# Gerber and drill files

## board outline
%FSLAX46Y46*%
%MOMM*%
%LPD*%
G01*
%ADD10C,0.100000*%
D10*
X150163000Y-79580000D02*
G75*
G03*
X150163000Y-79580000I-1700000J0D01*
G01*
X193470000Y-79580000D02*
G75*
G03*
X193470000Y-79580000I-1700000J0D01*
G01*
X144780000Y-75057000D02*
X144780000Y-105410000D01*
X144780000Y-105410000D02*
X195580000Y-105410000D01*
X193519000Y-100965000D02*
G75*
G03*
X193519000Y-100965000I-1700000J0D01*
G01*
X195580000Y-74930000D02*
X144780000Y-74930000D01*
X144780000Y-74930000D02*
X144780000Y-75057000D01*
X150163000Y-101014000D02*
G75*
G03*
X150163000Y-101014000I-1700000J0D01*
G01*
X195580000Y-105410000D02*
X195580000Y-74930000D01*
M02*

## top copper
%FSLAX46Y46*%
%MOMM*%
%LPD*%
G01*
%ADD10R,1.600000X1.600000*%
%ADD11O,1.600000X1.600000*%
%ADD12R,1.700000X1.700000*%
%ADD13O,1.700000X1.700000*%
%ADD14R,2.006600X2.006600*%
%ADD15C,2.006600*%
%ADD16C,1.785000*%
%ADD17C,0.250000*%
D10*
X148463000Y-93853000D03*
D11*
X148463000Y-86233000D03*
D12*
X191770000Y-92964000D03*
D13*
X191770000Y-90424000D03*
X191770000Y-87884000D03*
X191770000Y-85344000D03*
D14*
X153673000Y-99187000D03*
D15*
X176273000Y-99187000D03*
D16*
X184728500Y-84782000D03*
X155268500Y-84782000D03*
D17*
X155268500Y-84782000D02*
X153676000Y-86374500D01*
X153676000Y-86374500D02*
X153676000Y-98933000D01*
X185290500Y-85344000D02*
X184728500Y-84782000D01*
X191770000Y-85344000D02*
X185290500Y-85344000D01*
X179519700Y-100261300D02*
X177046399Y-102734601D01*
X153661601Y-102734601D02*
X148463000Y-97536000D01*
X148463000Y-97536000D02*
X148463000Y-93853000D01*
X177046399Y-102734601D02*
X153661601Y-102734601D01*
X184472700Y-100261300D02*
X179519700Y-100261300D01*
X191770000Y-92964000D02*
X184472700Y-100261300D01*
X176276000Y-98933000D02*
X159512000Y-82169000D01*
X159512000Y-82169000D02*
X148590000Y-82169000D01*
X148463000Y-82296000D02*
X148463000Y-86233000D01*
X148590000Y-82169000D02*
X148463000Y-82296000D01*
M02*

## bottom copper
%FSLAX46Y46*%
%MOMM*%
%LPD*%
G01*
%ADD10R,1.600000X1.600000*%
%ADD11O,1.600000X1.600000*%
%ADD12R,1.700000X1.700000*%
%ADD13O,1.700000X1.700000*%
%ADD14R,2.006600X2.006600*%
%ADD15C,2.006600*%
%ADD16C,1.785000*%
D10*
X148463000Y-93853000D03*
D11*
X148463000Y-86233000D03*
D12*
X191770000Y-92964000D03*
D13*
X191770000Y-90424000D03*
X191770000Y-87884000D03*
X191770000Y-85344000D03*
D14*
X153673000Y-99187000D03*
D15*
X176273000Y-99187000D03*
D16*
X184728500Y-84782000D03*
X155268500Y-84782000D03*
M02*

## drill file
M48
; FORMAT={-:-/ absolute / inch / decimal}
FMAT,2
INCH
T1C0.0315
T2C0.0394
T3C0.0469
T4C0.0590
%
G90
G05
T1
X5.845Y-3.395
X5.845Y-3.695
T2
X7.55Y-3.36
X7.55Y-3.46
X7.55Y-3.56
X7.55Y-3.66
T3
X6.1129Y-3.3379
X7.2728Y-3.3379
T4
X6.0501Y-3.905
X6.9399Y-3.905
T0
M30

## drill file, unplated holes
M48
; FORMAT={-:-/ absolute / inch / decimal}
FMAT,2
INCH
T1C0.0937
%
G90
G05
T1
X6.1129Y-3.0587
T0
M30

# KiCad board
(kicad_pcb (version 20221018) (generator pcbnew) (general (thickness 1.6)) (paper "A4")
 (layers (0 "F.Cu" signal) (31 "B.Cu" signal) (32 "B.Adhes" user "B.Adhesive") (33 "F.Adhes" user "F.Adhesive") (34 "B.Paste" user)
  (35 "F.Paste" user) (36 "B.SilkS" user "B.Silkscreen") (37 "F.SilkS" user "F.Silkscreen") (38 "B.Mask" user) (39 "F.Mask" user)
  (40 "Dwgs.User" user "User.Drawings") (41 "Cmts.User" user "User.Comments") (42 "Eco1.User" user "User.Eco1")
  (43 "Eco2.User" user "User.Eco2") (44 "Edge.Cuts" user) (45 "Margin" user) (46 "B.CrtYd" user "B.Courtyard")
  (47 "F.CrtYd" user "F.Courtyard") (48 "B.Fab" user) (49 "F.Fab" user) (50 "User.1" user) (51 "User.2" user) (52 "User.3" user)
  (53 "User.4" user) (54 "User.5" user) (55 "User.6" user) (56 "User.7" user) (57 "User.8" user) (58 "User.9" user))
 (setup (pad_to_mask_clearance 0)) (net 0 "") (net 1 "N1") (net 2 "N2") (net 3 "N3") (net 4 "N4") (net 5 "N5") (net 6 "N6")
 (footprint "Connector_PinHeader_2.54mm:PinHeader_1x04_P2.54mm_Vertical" (layer "F.Cu") (at 191.77 92.964 180)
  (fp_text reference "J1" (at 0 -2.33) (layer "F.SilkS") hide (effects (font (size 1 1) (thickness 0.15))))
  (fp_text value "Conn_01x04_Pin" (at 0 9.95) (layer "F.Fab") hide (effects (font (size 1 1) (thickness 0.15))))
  (pad "1" thru_hole rect (at 0 0 180) (size 1.7 1.7) (drill 1) (layers "*.Cu" "*.Mask") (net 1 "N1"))
  (pad "2" thru_hole oval (at 0 2.54 180) (size 1.7 1.7) (drill 1) (layers "*.Cu" "*.Mask") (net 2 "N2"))
  (pad "3" thru_hole oval (at 0 5.08 180) (size 1.7 1.7) (drill 1) (layers "*.Cu" "*.Mask") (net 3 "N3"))
  (pad "4" thru_hole oval (at 0 7.62 180) (size 1.7 1.7) (drill 1) (layers "*.Cu" "*.Mask") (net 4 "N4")))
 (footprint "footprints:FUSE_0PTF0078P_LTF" (layer "F.Cu") (at 153.673 99.187)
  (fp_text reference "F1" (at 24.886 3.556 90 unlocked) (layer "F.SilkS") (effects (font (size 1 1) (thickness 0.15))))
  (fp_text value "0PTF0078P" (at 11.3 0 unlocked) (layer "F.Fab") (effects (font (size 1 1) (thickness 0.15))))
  (pad "1" thru_hole rect (at 0 0) (size 2.0066 2.0066) (drill 1.4986) (layers "*.Cu" "*.Mask") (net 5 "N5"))
  (pad "2" thru_hole circle (at 22.6 0) (size 2.0066 2.0066) (drill 1.4986) (layers "*.Cu" "*.Mask") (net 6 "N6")))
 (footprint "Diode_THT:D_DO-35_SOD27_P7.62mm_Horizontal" (layer "F.Cu") (at 148.463 93.853 90)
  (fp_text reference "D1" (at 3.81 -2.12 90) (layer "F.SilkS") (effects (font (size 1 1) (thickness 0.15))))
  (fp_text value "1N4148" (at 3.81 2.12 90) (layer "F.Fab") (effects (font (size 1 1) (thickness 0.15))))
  (pad "1" thru_hole rect (at 0 0 90) (size 1.6 1.6) (drill 0.8) (layers "*.Cu" "*.Mask") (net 1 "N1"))
  (pad "2" thru_hole oval (at 7.62 0 90) (size 1.6 1.6) (drill 0.8) (layers "*.Cu" "*.Mask") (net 6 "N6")))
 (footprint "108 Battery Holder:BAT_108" (layer "F.Cu") (at 169.9985 84.782)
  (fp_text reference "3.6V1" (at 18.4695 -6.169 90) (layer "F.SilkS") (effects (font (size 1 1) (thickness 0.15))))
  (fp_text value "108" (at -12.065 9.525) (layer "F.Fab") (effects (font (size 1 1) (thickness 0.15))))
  (pad "" np_thru_hole circle (at -14.73 -7.09) (size 2.38 2.38) (drill 2.38) (layers "*.Cu" "*.Mask"))
  (pad "N" thru_hole circle (at 14.73 0) (size 1.785 1.785) (drill 1.19) (layers "*.Cu" "*.Mask") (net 4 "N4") (solder_mask_margin 0.102))
  (pad "P" thru_hole circle (at -14.73 0) (size 1.785 1.785) (drill 1.19) (layers "*.Cu" "*.Mask") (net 5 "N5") (solder_mask_margin 0.102)))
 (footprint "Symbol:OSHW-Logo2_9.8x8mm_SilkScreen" (layer "B.Cu") (at 183.515 98.933 180)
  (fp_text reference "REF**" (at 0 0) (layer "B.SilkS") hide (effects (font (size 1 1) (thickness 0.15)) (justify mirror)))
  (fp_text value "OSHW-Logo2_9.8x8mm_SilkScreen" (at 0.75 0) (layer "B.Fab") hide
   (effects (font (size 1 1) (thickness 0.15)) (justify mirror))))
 (gr_circle (center 148.463 79.58) (end 150.163 79.58) (stroke (width 0.1) (type default)) (fill none) (layer "Edge.Cuts"))
 (gr_circle (center 191.77 79.58) (end 193.47 79.58) (stroke (width 0.1) (type default)) (fill none) (layer "Edge.Cuts"))
 (gr_line (start 144.78 75.057) (end 144.78 105.41) (stroke (width 0.1) (type default)) (layer "Edge.Cuts"))
 (gr_line (start 144.78 105.41) (end 195.58 105.41) (stroke (width 0.1) (type default)) (layer "Edge.Cuts"))
 (gr_circle (center 191.819 100.965) (end 193.519 100.965) (stroke (width 0.1) (type default)) (fill none) (layer "Edge.Cuts"))
 (gr_line (start 195.58 74.93) (end 144.78 74.93) (stroke (width 0.1) (type default)) (layer "Edge.Cuts"))
 (gr_line (start 144.78 74.93) (end 144.78 75.057) (stroke (width 0.1) (type default)) (layer "Edge.Cuts"))
 (gr_circle (center 148.463 101.014) (end 150.163 101.014) (stroke (width 0.1) (type default)) (fill none) (layer "Edge.Cuts"))
 (gr_line (start 195.58 105.41) (end 195.58 74.93) (stroke (width 0.1) (type default)) (layer "Edge.Cuts"))
 (segment (start 155.2685 84.782) (end 153.676 86.3745) (width 0.25) (layer "F.Cu") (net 5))
 (segment (start 153.676 86.3745) (end 153.676 98.933) (width 0.25) (layer "F.Cu") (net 5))
 (segment (start 185.2905 85.344) (end 184.7285 84.782) (width 0.25) (layer "F.Cu") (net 4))
 (segment (start 191.77 85.344) (end 185.2905 85.344) (width 0.25) (layer "F.Cu") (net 4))
 (segment (start 179.5197 100.2613) (end 177.046399 102.734601) (width 0.25) (layer "F.Cu") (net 1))
 (segment (start 153.661601 102.734601) (end 148.463 97.536) (width 0.25) (layer "F.Cu") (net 1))
 (segment (start 148.463 97.536) (end 148.463 93.853) (width 0.25) (layer "F.Cu") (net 1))
 (segment (start 177.046399 102.734601) (end 153.661601 102.734601) (width 0.25) (layer "F.Cu") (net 1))
 (segment (start 184.4727 100.2613) (end 179.5197 100.2613) (width 0.25) (layer "F.Cu") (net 1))
 (segment (start 191.77 92.964) (end 184.4727 100.2613) (width 0.25) (layer "F.Cu") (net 1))
 (segment (start 176.276 98.933) (end 159.512 82.169) (width 0.25) (layer "F.Cu") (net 6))
 (segment (start 159.512 82.169) (end 148.59 82.169) (width 0.25) (layer "F.Cu") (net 6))
 (segment (start 148.463 82.296) (end 148.463 86.233) (width 0.25) (layer "F.Cu") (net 6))
 (segment (start 148.59 82.169) (end 148.463 82.296) (width 0.25) (layer "F.Cu") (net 6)))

